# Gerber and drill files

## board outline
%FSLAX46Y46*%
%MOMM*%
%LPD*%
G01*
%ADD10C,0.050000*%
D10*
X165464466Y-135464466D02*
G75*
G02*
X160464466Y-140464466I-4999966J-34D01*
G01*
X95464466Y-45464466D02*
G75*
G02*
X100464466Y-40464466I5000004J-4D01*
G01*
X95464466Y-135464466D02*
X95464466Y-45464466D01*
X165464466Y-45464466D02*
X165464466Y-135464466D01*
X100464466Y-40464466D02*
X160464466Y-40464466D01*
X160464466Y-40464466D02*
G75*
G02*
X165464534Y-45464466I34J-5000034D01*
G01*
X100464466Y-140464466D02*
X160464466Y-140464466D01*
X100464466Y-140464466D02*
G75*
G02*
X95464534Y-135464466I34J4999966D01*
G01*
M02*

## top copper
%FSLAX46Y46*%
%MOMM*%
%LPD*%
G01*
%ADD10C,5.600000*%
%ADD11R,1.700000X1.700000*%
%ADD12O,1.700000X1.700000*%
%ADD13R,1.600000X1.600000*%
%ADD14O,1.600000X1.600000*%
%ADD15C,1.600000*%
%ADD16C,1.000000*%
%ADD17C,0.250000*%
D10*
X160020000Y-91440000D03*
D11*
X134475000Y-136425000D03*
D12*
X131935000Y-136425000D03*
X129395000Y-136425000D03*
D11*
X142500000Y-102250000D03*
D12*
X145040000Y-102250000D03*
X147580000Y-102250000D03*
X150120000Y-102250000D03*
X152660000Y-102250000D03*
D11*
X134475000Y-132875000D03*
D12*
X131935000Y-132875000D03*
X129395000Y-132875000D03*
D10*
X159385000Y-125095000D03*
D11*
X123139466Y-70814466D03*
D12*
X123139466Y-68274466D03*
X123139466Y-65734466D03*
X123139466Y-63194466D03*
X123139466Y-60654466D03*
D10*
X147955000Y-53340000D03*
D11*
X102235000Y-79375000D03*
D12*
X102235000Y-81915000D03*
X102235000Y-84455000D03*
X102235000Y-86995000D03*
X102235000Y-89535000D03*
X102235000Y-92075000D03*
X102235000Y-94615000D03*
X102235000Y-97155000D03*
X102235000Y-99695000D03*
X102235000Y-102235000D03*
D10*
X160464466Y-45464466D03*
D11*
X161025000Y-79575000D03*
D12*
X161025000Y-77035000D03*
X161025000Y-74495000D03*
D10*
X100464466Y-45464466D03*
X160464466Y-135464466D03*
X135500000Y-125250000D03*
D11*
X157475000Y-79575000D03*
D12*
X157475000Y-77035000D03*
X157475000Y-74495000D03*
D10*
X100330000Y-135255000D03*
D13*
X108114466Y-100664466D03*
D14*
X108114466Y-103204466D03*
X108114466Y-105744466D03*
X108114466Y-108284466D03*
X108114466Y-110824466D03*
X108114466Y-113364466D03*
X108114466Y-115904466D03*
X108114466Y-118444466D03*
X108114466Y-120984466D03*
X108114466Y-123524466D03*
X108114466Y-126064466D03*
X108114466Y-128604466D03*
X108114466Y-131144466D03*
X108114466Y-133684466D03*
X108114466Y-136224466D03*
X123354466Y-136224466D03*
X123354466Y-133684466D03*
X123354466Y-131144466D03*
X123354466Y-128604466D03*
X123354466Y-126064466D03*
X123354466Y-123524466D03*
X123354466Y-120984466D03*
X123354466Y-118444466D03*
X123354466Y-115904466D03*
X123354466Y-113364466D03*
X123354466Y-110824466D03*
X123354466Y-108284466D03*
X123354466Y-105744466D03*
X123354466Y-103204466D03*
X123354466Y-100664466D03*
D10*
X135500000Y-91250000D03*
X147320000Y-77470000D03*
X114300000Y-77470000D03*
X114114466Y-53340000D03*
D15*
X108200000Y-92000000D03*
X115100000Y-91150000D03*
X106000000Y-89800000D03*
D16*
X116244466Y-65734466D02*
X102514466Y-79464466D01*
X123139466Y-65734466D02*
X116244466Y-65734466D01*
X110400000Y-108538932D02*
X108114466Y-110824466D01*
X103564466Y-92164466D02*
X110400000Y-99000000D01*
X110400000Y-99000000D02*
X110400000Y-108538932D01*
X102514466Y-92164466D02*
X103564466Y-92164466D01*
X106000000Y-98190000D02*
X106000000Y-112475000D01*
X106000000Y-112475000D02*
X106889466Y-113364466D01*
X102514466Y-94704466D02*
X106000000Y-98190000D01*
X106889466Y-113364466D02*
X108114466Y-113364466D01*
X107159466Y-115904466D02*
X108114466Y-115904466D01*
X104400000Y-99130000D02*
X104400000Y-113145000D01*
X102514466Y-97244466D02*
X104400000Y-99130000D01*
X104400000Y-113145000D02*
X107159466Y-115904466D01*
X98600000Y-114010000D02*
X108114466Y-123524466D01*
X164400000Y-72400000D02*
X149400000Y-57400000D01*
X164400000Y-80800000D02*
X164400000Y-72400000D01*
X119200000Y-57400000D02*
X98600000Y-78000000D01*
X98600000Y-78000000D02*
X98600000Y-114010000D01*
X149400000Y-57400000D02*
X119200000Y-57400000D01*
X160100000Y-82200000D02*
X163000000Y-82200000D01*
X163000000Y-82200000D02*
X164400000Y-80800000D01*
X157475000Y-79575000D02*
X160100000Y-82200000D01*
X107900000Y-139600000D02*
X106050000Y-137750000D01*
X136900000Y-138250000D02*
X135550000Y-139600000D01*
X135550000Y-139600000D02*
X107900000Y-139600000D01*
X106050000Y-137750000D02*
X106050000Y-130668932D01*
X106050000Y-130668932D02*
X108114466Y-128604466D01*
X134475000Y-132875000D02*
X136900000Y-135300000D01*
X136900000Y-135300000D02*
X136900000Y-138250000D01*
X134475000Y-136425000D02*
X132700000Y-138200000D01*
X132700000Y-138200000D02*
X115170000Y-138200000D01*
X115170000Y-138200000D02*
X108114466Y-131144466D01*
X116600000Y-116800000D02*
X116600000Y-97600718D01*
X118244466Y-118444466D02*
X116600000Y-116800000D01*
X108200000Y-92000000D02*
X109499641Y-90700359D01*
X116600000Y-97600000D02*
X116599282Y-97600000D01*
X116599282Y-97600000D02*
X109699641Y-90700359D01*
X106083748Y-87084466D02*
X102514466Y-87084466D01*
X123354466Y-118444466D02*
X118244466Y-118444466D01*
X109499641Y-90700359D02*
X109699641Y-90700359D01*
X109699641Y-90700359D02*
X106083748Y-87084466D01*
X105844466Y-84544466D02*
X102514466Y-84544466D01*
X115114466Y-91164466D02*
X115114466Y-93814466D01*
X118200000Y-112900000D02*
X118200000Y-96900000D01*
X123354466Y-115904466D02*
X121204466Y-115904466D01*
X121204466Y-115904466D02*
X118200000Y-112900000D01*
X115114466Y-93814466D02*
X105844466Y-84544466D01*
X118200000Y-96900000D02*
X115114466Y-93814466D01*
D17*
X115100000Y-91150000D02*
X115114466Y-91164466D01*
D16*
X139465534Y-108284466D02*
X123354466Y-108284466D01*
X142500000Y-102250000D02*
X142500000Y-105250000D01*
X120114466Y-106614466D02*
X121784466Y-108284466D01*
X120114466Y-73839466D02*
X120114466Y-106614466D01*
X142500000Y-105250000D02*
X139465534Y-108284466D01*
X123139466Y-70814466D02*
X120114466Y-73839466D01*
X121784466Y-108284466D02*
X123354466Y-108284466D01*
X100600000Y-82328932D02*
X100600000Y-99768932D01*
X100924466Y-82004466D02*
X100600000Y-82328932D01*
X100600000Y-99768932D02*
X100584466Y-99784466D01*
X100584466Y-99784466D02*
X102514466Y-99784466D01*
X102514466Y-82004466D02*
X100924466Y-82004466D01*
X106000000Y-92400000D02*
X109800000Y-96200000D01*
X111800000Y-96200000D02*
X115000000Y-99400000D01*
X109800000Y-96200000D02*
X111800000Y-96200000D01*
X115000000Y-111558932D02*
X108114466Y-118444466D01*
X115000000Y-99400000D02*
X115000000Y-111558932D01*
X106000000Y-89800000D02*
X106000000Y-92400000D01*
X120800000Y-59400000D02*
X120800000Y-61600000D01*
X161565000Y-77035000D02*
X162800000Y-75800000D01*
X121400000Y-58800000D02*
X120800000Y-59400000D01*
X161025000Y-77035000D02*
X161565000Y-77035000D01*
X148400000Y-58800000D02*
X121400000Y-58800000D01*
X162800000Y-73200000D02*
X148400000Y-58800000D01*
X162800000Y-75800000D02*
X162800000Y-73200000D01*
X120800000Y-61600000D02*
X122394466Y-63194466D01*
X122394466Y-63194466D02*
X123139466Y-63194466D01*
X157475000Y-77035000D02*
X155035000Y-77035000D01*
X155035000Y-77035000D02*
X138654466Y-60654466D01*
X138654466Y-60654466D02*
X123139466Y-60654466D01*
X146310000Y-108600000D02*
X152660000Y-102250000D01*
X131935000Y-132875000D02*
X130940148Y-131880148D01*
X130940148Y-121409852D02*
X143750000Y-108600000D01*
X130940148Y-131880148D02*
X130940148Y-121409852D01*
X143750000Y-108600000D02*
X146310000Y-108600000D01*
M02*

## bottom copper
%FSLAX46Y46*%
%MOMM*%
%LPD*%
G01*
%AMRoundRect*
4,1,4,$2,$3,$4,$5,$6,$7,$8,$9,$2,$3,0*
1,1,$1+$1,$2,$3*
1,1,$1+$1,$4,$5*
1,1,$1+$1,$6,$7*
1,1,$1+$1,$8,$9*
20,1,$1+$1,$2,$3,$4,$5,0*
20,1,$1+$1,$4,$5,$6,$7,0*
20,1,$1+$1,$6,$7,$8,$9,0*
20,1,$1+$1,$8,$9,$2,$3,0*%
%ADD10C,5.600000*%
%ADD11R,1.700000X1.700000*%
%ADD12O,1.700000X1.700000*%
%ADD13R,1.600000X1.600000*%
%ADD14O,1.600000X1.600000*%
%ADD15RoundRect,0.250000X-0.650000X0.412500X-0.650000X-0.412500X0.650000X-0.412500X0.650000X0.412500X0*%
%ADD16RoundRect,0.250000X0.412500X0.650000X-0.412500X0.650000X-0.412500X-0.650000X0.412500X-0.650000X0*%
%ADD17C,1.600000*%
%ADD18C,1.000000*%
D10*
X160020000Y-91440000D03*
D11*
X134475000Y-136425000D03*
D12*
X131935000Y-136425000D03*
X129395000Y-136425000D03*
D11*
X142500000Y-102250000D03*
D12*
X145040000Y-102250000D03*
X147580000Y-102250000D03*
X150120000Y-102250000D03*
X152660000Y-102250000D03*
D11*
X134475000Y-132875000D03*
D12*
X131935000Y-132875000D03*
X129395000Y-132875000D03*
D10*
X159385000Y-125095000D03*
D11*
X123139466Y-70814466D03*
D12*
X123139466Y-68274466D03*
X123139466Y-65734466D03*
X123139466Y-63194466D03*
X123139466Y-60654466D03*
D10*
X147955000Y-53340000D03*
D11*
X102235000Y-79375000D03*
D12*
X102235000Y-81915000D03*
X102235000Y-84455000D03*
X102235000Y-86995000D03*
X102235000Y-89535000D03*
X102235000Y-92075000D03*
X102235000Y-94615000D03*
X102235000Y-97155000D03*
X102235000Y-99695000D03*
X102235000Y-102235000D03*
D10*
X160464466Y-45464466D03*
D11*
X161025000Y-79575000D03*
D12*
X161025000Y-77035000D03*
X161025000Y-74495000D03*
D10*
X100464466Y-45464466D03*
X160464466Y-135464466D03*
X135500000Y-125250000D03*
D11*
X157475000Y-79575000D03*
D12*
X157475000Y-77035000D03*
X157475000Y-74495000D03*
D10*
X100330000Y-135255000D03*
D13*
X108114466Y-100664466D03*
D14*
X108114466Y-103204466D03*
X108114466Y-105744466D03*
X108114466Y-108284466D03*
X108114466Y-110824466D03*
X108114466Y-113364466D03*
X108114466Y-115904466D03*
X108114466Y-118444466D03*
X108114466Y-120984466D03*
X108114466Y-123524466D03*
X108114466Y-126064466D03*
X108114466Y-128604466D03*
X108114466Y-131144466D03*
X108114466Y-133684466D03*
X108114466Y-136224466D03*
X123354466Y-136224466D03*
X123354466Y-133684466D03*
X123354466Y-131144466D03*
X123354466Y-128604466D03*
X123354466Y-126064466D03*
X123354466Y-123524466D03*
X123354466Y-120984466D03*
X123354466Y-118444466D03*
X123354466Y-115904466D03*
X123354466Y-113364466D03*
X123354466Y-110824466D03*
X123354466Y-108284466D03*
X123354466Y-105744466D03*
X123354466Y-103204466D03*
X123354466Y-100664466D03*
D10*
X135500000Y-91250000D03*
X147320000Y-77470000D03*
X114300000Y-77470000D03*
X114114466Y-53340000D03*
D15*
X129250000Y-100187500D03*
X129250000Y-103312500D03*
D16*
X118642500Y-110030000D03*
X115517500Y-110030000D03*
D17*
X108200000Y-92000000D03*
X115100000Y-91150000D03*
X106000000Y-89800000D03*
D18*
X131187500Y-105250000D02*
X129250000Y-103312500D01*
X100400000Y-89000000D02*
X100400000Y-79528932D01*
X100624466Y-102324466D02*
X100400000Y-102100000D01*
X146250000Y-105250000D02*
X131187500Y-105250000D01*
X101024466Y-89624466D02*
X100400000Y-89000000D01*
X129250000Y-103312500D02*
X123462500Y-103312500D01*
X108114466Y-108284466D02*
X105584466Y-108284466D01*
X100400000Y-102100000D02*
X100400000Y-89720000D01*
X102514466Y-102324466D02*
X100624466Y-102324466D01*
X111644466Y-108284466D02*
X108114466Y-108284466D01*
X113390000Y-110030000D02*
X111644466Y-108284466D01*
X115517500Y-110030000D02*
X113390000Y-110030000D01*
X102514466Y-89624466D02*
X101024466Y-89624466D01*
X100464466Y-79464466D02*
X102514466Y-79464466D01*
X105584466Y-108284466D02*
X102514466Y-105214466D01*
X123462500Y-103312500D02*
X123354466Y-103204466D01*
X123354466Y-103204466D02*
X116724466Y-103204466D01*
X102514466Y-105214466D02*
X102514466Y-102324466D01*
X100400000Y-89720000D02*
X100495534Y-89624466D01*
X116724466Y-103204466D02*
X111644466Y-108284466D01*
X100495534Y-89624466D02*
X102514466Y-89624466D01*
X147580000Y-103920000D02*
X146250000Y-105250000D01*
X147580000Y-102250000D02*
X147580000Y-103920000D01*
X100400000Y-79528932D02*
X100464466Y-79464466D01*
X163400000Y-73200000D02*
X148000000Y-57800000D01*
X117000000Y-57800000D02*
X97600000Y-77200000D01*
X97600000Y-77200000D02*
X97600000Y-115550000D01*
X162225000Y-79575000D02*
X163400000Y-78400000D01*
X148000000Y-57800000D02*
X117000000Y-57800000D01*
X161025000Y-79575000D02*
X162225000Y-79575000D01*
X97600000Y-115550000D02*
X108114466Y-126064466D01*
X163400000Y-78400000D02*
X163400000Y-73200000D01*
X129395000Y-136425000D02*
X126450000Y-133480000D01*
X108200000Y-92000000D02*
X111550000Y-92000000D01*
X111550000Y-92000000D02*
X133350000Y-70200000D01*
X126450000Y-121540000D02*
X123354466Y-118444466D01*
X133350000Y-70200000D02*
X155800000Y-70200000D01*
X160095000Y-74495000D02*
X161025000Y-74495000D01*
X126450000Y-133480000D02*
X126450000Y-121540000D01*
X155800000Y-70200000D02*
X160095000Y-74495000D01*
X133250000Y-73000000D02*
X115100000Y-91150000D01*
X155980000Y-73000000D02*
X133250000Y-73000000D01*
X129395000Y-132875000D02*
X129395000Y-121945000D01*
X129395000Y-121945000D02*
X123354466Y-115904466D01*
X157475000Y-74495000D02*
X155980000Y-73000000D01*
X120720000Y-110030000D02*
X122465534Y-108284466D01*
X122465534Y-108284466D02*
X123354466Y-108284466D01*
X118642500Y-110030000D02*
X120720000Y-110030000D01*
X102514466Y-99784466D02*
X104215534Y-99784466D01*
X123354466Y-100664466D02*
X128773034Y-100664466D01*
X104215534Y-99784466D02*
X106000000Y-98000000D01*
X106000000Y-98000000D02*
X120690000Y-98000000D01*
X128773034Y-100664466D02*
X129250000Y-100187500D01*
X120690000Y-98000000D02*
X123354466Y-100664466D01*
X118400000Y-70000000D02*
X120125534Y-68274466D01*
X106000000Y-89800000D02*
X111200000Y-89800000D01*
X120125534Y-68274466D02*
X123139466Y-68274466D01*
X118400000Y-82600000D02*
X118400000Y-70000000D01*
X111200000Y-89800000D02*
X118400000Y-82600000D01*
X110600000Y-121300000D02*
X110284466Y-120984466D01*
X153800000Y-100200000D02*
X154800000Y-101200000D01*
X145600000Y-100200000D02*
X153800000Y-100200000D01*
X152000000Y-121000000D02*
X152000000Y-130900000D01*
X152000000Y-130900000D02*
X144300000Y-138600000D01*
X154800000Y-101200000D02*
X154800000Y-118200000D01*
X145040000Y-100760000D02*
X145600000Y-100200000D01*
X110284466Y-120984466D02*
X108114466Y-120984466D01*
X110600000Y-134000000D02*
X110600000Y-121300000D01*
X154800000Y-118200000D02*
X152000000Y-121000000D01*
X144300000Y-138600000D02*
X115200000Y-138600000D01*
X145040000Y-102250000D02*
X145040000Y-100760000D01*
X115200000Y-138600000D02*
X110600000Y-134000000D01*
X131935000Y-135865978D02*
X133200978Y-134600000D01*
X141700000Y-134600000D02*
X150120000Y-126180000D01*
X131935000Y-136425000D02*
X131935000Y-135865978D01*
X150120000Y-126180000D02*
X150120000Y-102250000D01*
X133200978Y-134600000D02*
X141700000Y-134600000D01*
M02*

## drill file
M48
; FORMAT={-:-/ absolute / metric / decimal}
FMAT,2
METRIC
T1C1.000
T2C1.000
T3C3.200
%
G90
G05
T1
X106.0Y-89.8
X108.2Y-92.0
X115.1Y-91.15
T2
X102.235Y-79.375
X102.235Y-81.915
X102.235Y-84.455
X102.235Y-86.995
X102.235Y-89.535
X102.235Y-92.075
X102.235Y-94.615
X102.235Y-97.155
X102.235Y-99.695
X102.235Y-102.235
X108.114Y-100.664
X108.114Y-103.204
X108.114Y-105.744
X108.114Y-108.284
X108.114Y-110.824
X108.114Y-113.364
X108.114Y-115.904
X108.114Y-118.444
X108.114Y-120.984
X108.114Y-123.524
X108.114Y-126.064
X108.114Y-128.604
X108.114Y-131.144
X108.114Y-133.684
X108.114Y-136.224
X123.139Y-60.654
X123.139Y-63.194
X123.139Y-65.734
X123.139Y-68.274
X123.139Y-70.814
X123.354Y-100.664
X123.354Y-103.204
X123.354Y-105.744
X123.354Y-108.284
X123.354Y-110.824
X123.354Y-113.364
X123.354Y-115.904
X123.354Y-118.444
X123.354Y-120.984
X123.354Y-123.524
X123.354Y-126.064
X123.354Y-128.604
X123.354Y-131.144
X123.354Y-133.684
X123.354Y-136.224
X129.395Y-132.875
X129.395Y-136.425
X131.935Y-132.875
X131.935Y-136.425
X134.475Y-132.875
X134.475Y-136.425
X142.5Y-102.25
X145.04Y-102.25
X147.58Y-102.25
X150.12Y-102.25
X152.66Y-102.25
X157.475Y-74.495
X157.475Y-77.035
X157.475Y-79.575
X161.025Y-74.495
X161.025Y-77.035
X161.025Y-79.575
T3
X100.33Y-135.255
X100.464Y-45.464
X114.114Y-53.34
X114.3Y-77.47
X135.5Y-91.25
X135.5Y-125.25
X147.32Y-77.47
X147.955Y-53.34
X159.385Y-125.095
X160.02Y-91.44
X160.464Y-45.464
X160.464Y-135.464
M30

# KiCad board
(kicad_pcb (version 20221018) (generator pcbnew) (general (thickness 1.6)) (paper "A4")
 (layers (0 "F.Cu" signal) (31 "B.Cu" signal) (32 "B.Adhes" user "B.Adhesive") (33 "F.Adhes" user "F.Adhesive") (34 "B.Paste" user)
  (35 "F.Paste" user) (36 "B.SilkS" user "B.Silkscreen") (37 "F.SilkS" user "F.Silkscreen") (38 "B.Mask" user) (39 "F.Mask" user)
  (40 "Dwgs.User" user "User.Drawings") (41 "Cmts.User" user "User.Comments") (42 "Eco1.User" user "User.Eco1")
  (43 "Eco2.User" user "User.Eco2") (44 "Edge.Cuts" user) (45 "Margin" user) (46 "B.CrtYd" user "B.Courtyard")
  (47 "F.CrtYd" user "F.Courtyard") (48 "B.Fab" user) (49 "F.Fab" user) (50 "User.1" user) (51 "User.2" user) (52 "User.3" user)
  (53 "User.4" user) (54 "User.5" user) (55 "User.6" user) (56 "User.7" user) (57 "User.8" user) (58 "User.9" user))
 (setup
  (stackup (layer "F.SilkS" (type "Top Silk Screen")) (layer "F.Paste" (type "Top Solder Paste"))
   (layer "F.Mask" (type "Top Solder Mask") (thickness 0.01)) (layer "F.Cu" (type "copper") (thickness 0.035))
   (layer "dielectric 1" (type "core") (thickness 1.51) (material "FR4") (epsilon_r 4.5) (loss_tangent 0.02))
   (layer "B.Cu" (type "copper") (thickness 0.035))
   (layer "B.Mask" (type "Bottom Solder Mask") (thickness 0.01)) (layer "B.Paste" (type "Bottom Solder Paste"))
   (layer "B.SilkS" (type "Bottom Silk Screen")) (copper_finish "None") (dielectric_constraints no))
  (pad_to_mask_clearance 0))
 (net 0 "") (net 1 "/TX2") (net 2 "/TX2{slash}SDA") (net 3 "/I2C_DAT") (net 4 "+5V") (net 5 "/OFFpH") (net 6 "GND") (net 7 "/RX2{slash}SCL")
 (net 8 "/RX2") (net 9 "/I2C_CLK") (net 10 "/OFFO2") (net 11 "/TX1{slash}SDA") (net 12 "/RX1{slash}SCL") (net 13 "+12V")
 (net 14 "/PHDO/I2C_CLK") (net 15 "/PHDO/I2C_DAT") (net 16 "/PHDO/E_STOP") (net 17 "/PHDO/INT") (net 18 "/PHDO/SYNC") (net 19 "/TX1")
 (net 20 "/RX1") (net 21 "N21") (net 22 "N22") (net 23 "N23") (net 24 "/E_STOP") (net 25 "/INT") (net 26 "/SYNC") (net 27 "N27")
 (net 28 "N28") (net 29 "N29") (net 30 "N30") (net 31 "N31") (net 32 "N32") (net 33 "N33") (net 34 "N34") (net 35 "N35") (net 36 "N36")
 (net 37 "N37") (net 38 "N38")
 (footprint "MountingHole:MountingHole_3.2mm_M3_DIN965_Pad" (layer "F.Cu") (at 160.02 91.44)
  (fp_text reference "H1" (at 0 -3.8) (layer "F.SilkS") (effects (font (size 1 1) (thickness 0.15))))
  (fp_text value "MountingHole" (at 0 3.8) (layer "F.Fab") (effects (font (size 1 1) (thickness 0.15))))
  (pad "1" thru_hole circle (at 0 0) (size 5.6 5.6) (drill 3.2) (layers "*.Cu" "*.Mask")))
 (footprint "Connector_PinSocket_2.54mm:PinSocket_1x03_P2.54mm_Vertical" (layer "F.Cu") (at 134.475 136.425 -90)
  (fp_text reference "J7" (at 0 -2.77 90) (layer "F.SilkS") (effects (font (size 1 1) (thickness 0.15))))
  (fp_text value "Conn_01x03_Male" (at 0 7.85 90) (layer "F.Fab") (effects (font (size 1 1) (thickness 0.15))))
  (pad "1" thru_hole rect (at 0 0 270) (size 1.7 1.7) (drill 1) (layers "*.Cu" "*.Mask") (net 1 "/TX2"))
  (pad "2" thru_hole oval (at 0 2.54 270) (size 1.7 1.7) (drill 1) (layers "*.Cu" "*.Mask") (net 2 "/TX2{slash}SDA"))
  (pad "3" thru_hole oval (at 0 5.08 270) (size 1.7 1.7) (drill 1) (layers "*.Cu" "*.Mask") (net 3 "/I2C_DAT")))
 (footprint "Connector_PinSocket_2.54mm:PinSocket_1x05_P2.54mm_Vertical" (layer "F.Cu") (at 142.5 102.25 90)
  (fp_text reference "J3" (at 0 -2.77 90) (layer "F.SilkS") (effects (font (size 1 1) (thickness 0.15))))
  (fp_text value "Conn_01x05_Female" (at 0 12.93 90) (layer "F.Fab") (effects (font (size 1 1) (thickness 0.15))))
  (pad "1" thru_hole rect (at 0 0 90) (size 1.7 1.7) (drill 1) (layers "*.Cu" "*.Mask") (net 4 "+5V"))
  (pad "2" thru_hole oval (at 0 2.54 90) (size 1.7 1.7) (drill 1) (layers "*.Cu" "*.Mask") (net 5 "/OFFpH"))
  (pad "3" thru_hole oval (at 0 5.08 90) (size 1.7 1.7) (drill 1) (layers "*.Cu" "*.Mask") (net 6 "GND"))
  (pad "4" thru_hole oval (at 0 7.62 90) (size 1.7 1.7) (drill 1) (layers "*.Cu" "*.Mask") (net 2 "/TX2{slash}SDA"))
  (pad "5" thru_hole oval (at 0 10.16 90) (size 1.7 1.7) (drill 1) (layers "*.Cu" "*.Mask") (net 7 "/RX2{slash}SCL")))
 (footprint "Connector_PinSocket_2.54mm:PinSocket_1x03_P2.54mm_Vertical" (layer "F.Cu") (at 134.475 132.875 -90)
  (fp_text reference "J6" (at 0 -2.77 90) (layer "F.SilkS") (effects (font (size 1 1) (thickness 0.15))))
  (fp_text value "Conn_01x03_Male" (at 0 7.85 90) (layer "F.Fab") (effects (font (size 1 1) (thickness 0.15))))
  (pad "1" thru_hole rect (at 0 0 270) (size 1.7 1.7) (drill 1) (layers "*.Cu" "*.Mask") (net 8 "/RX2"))
  (pad "2" thru_hole oval (at 0 2.54 270) (size 1.7 1.7) (drill 1) (layers "*.Cu" "*.Mask") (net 7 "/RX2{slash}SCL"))
  (pad "3" thru_hole oval (at 0 5.08 270) (size 1.7 1.7) (drill 1) (layers "*.Cu" "*.Mask") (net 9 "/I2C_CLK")))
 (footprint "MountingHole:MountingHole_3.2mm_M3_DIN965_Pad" (layer "F.Cu") (at 159.385 125.095)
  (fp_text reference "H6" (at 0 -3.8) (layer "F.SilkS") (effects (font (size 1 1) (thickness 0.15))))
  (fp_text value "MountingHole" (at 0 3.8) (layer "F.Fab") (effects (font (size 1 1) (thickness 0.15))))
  (pad "1" thru_hole circle (at 0 0) (size 5.6 5.6) (drill 3.2) (layers "*.Cu" "*.Mask")))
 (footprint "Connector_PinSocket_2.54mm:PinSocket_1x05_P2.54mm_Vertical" (layer "F.Cu") (at 123.139466 70.814466 180)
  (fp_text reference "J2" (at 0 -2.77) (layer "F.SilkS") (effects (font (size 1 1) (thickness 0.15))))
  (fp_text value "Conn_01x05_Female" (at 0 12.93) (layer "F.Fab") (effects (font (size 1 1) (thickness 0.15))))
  (pad "1" thru_hole rect (at 0 0 180) (size 1.7 1.7) (drill 1) (layers "*.Cu" "*.Mask") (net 4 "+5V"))
  (pad "2" thru_hole oval (at 0 2.54 180) (size 1.7 1.7) (drill 1) (layers "*.Cu" "*.Mask") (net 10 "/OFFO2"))
  (pad "3" thru_hole oval (at 0 5.08 180) (size 1.7 1.7) (drill 1) (layers "*.Cu" "*.Mask") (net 6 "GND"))
  (pad "4" thru_hole oval (at 0 7.62 180) (size 1.7 1.7) (drill 1) (layers "*.Cu" "*.Mask") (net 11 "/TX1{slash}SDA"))
  (pad "5" thru_hole oval (at 0 10.16 180) (size 1.7 1.7) (drill 1) (layers "*.Cu" "*.Mask") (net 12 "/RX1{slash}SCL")))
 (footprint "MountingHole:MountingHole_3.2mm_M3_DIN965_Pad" (layer "F.Cu") (at 147.955 53.34)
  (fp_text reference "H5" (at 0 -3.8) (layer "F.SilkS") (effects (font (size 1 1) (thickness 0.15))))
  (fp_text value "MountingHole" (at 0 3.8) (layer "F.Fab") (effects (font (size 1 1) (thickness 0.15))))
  (pad "1" thru_hole circle (at 0 0) (size 5.6 5.6) (drill 3.2) (layers "*.Cu" "*.Mask")))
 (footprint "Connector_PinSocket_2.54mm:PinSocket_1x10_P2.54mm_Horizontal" (layer "F.Cu") (at 102.235 79.375)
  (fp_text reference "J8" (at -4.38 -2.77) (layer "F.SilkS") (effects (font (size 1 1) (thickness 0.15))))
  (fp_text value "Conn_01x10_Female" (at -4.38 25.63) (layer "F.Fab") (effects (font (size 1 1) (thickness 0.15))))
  (pad "1" thru_hole rect (at 0 0) (size 1.7 1.7) (drill 1) (layers "*.Cu" "*.Mask") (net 6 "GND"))
  (pad "2" thru_hole oval (at 0 2.54) (size 1.7 1.7) (drill 1) (layers "*.Cu" "*.Mask") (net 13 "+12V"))
  (pad "3" thru_hole oval (at 0 5.08) (size 1.7 1.7) (drill 1) (layers "*.Cu" "*.Mask") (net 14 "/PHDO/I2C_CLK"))
  (pad "4" thru_hole oval (at 0 7.62) (size 1.7 1.7) (drill 1) (layers "*.Cu" "*.Mask") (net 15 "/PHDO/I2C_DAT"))
  (pad "5" thru_hole oval (at 0 10.16) (size 1.7 1.7) (drill 1) (layers "*.Cu" "*.Mask") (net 6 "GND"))
  (pad "6" thru_hole oval (at 0 12.7) (size 1.7 1.7) (drill 1) (layers "*.Cu" "*.Mask") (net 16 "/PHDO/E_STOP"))
  (pad "7" thru_hole oval (at 0 15.24) (size 1.7 1.7) (drill 1) (layers "*.Cu" "*.Mask") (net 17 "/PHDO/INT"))
  (pad "8" thru_hole oval (at 0 17.78) (size 1.7 1.7) (drill 1) (layers "*.Cu" "*.Mask") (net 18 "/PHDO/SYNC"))
  (pad "9" thru_hole oval (at 0 20.32) (size 1.7 1.7) (drill 1) (layers "*.Cu" "*.Mask") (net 13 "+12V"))
  (pad "10" thru_hole oval (at 0 22.86) (size 1.7 1.7) (drill 1) (layers "*.Cu" "*.Mask") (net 6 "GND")))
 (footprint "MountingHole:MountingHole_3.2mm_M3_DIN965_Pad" (layer "F.Cu") (at 160.464466 45.464466)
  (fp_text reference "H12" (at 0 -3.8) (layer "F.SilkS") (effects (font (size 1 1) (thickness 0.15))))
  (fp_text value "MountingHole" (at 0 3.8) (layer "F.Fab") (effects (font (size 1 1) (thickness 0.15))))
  (pad "1" thru_hole circle (at 0 0) (size 5.6 5.6) (drill 3.2) (layers "*.Cu" "*.Mask")))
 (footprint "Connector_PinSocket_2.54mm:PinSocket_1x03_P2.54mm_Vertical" (layer "F.Cu") (at 161.025 79.575 180)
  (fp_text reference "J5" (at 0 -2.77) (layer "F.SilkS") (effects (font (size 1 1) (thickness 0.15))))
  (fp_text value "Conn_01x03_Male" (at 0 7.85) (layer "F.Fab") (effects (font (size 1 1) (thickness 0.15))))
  (pad "1" thru_hole rect (at 0 0 180) (size 1.7 1.7) (drill 1) (layers "*.Cu" "*.Mask") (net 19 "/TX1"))
  (pad "2" thru_hole oval (at 0 2.54 180) (size 1.7 1.7) (drill 1) (layers "*.Cu" "*.Mask") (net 11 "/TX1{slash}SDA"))
  (pad "3" thru_hole oval (at 0 5.08 180) (size 1.7 1.7) (drill 1) (layers "*.Cu" "*.Mask") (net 3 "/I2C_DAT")))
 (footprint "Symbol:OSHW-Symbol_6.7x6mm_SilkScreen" (layer "F.Cu") (at 109.515 44.979 180)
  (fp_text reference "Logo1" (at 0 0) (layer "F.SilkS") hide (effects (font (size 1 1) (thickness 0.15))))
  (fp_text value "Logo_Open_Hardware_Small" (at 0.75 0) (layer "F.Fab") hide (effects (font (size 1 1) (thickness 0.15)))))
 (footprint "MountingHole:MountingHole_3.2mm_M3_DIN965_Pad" (layer "F.Cu") (at 100.464466 45.464466)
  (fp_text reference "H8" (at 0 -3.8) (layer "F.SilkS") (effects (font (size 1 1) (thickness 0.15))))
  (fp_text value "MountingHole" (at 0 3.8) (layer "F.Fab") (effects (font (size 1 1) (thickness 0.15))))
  (pad "1" thru_hole circle (at 0 0) (size 5.6 5.6) (drill 3.2) (layers "*.Cu" "*.Mask")))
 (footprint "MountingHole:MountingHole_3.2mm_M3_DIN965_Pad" (layer "F.Cu") (at 160.464466 135.464466)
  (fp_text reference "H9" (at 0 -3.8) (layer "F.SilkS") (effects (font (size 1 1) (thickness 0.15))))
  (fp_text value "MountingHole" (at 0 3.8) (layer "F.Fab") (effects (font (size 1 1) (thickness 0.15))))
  (pad "1" thru_hole circle (at 0 0) (size 5.6 5.6) (drill 3.2) (layers "*.Cu" "*.Mask")))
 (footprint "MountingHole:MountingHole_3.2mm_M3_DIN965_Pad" (layer "F.Cu") (at 135.5 125.25 90)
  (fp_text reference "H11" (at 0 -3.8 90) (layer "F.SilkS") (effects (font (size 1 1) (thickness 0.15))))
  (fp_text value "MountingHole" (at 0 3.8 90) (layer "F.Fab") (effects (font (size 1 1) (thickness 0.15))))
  (pad "1" thru_hole circle (at 0 0 90) (size 5.6 5.6) (drill 3.2) (layers "*.Cu" "*.Mask")))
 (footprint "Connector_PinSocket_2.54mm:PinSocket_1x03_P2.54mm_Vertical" (layer "F.Cu") (at 157.475 79.575 180)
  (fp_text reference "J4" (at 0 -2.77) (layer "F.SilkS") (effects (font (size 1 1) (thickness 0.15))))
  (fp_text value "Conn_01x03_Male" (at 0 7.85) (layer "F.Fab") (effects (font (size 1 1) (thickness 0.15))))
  (pad "1" thru_hole rect (at 0 0 180) (size 1.7 1.7) (drill 1) (layers "*.Cu" "*.Mask") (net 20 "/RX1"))
  (pad "2" thru_hole oval (at 0 2.54 180) (size 1.7 1.7) (drill 1) (layers "*.Cu" "*.Mask") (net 12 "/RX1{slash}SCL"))
  (pad "3" thru_hole oval (at 0 5.08 180) (size 1.7 1.7) (drill 1) (layers "*.Cu" "*.Mask") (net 9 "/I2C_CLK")))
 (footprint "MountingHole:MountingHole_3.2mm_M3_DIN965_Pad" (layer "F.Cu") (at 100.33 135.255)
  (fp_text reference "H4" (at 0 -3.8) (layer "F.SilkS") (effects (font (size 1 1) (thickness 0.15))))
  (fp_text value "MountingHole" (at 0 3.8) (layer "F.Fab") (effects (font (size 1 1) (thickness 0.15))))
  (pad "1" thru_hole circle (at 0 0) (size 5.6 5.6) (drill 3.2) (layers "*.Cu" "*.Mask")))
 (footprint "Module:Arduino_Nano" (layer "F.Cu") (at 108.114466 100.664466)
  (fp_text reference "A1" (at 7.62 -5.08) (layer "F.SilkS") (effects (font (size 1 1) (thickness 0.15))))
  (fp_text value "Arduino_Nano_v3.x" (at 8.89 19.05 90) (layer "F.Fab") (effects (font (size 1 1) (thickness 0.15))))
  (pad "1" thru_hole rect (at 0 0) (size 1.6 1.6) (drill 1) (layers "*.Cu" "*.Mask") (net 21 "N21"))
  (pad "2" thru_hole oval (at 0 2.54) (size 1.6 1.6) (drill 1) (layers "*.Cu" "*.Mask") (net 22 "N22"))
  (pad "3" thru_hole oval (at 0 5.08) (size 1.6 1.6) (drill 1) (layers "*.Cu" "*.Mask") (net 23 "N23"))
  (pad "4" thru_hole oval (at 0 7.62) (size 1.6 1.6) (drill 1) (layers "*.Cu" "*.Mask") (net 6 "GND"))
  (pad "5" thru_hole oval (at 0 10.16) (size 1.6 1.6) (drill 1) (layers "*.Cu" "*.Mask") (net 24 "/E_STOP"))
  (pad "6" thru_hole oval (at 0 12.7) (size 1.6 1.6) (drill 1) (layers "*.Cu" "*.Mask") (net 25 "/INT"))
  (pad "7" thru_hole oval (at 0 15.24) (size 1.6 1.6) (drill 1) (layers "*.Cu" "*.Mask") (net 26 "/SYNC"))
  (pad "8" thru_hole oval (at 0 17.78) (size 1.6 1.6) (drill 1) (layers "*.Cu" "*.Mask") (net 10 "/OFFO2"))
  (pad "9" thru_hole oval (at 0 20.32) (size 1.6 1.6) (drill 1) (layers "*.Cu" "*.Mask") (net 5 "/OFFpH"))
  (pad "10" thru_hole oval (at 0 22.86) (size 1.6 1.6) (drill 1) (layers "*.Cu" "*.Mask") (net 20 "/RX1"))
  (pad "11" thru_hole oval (at 0 25.4) (size 1.6 1.6) (drill 1) (layers "*.Cu" "*.Mask") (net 19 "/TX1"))
  (pad "12" thru_hole oval (at 0 27.94) (size 1.6 1.6) (drill 1) (layers "*.Cu" "*.Mask") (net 8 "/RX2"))
  (pad "13" thru_hole oval (at 0 30.48) (size 1.6 1.6) (drill 1) (layers "*.Cu" "*.Mask") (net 1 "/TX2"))
  (pad "14" thru_hole oval (at 0 33.02) (size 1.6 1.6) (drill 1) (layers "*.Cu" "*.Mask") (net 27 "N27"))
  (pad "15" thru_hole oval (at 0 35.56) (size 1.6 1.6) (drill 1) (layers "*.Cu" "*.Mask") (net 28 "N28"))
  (pad "16" thru_hole oval (at 15.24 35.56) (size 1.6 1.6) (drill 1) (layers "*.Cu" "*.Mask") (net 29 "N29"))
  (pad "17" thru_hole oval (at 15.24 33.02) (size 1.6 1.6) (drill 1) (layers "*.Cu" "*.Mask") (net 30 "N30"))
  (pad "18" thru_hole oval (at 15.24 30.48) (size 1.6 1.6) (drill 1) (layers "*.Cu" "*.Mask") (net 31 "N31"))
  (pad "19" thru_hole oval (at 15.24 27.94) (size 1.6 1.6) (drill 1) (layers "*.Cu" "*.Mask") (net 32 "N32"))
  (pad "20" thru_hole oval (at 15.24 25.4) (size 1.6 1.6) (drill 1) (layers "*.Cu" "*.Mask") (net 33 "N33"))
  (pad "21" thru_hole oval (at 15.24 22.86) (size 1.6 1.6) (drill 1) (layers "*.Cu" "*.Mask") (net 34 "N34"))
  (pad "22" thru_hole oval (at 15.24 20.32) (size 1.6 1.6) (drill 1) (layers "*.Cu" "*.Mask") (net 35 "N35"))
  (pad "23" thru_hole oval (at 15.24 17.78) (size 1.6 1.6) (drill 1) (layers "*.Cu" "*.Mask") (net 3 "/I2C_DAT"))
  (pad "24" thru_hole oval (at 15.24 15.24) (size 1.6 1.6) (drill 1) (layers "*.Cu" "*.Mask") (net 9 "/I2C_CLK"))
  (pad "25" thru_hole oval (at 15.24 12.7) (size 1.6 1.6) (drill 1) (layers "*.Cu" "*.Mask") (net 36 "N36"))
  (pad "26" thru_hole oval (at 15.24 10.16) (size 1.6 1.6) (drill 1) (layers "*.Cu" "*.Mask") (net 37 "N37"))
  (pad "27" thru_hole oval (at 15.24 7.62) (size 1.6 1.6) (drill 1) (layers "*.Cu" "*.Mask") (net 4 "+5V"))
  (pad "28" thru_hole oval (at 15.24 5.08) (size 1.6 1.6) (drill 1) (layers "*.Cu" "*.Mask") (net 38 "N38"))
  (pad "29" thru_hole oval (at 15.24 2.54) (size 1.6 1.6) (drill 1) (layers "*.Cu" "*.Mask") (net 6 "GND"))
  (pad "30" thru_hole oval (at 15.24 0) (size 1.6 1.6) (drill 1) (layers "*.Cu" "*.Mask") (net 13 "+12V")))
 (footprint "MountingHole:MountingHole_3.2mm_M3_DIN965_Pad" (layer "F.Cu") (at 135.5 91.25 90)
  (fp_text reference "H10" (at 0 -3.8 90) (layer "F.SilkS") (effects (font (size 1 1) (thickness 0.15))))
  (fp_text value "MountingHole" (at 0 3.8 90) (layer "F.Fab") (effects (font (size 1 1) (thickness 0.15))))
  (pad "1" thru_hole circle (at 0 0 90) (size 5.6 5.6) (drill 3.2) (layers "*.Cu" "*.Mask")))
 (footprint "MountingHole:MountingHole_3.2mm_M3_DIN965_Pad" (layer "F.Cu") (at 147.32 77.47)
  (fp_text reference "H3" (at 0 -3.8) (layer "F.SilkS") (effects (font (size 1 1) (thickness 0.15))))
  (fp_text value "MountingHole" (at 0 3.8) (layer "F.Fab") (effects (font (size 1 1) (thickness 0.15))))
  (pad "1" thru_hole circle (at 0 0) (size 5.6 5.6) (drill 3.2) (layers "*.Cu" "*.Mask")))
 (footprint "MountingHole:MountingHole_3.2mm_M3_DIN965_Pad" (layer "F.Cu") (at 114.3 77.47)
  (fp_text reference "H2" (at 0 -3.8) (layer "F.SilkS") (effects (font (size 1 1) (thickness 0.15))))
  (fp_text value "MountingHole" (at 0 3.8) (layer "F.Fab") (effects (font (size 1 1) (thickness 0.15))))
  (pad "1" thru_hole circle (at 0 0) (size 5.6 5.6) (drill 3.2) (layers "*.Cu" "*.Mask")))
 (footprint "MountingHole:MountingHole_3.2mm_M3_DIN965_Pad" (layer "F.Cu") (at 114.114466 53.34)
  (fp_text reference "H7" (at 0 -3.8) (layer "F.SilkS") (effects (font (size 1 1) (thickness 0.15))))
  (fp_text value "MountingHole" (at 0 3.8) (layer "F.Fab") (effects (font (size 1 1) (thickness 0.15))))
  (pad "1" thru_hole circle (at 0 0) (size 5.6 5.6) (drill 3.2) (layers "*.Cu" "*.Mask")))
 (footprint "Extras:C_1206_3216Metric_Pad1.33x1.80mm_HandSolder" (layer "B.Cu") (at 129.25 101.75 -90)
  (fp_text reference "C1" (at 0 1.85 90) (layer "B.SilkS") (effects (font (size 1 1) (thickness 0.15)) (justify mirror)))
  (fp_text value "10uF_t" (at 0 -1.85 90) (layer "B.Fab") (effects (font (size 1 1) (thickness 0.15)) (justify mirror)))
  (pad "1" smd roundrect (at -1.5625 0 270) (size 1.325 1.8) (layers "B.Cu" "B.Paste" "B.Mask") (roundrect_rratio 0.1886792453)
   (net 13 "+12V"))
  (pad "2" smd roundrect (at 1.5625 0 270) (size 1.325 1.8) (layers "B.Cu" "B.Paste" "B.Mask") (roundrect_rratio 0.1886792453) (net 6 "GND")))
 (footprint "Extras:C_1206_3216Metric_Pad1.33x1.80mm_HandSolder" (layer "B.Cu") (at 117.08 110.03 180)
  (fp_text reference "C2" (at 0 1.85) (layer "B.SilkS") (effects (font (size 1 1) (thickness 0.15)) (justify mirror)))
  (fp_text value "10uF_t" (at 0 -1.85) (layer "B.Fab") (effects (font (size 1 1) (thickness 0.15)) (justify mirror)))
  (pad "1" smd roundrect (at -1.5625 0 180) (size 1.325 1.8) (layers "B.Cu" "B.Paste" "B.Mask") (roundrect_rratio 0.1886792453)
   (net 4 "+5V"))
  (pad "2" smd roundrect (at 1.5625 0 180) (size 1.325 1.8) (layers "B.Cu" "B.Paste" "B.Mask") (roundrect_rratio 0.1886792453) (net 6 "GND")))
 (gr_arc (start 165.464466 135.464466) (mid 164 139) (end 160.464466 140.464466) (stroke (width 0.05) (type solid)) (layer "Edge.Cuts"))
 (gr_arc (start 95.464466 45.464466) (mid 96.928932 41.928932) (end 100.464466 40.464466) (stroke (width 0.05) (type solid))
  (layer "Edge.Cuts"))
 (gr_line (start 95.464466 135.464466) (end 95.464466 45.464466) (stroke (width 0.05) (type solid)) (layer "Edge.Cuts"))
 (gr_line (start 165.464466 45.464466) (end 165.464466 135.464466) (stroke (width 0.05) (type solid)) (layer "Edge.Cuts"))
 (gr_line (start 100.464466 40.464466) (end 160.464466 40.464466) (stroke (width 0.05) (type solid)) (layer "Edge.Cuts"))
 (gr_arc (start 160.464466 40.464466) (mid 164 41.928932) (end 165.464466 45.464466) (stroke (width 0.05) (type solid)) (layer "Edge.Cuts"))
 (gr_line (start 100.464466 140.464466) (end 160.464466 140.464466) (stroke (width 0.05) (type solid)) (layer "Edge.Cuts"))
 (gr_arc (start 100.464466 140.464466) (mid 96.928932 139) (end 95.464466 135.464466) (stroke (width 0.05) (type solid)) (layer "Edge.Cuts"))
 (segment (start 116.244466 65.734466) (end 102.514466 79.464466) (width 1) (layer "F.Cu") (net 6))
 (segment (start 123.139466 65.734466) (end 116.244466 65.734466) (width 1) (layer "F.Cu") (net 6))
 (segment (start 131.1875 105.25) (end 129.25 103.3125) (width 1) (layer "B.Cu") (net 6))
 (segment (start 100.4 89) (end 100.4 79.528932) (width 1) (layer "B.Cu") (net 6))
 (segment (start 100.624466 102.324466) (end 100.4 102.1) (width 1) (layer "B.Cu") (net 6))
 (segment (start 146.25 105.25) (end 131.1875 105.25) (width 1) (layer "B.Cu") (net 6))
 (segment (start 101.024466 89.624466) (end 100.4 89) (width 1) (layer "B.Cu") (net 6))
 (segment (start 129.25 103.3125) (end 123.4625 103.3125) (width 1) (layer "B.Cu") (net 6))
 (segment (start 108.114466 108.284466) (end 105.584466 108.284466) (width 1) (layer "B.Cu") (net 6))
 (segment (start 100.4 102.1) (end 100.4 89.72) (width 1) (layer "B.Cu") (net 6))
 (segment (start 102.514466 102.324466) (end 100.624466 102.324466) (width 1) (layer "B.Cu") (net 6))
 (segment (start 111.644466 108.284466) (end 108.114466 108.284466) (width 1) (layer "B.Cu") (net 6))
 (segment (start 113.39 110.03) (end 111.644466 108.284466) (width 1) (layer "B.Cu") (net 6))
 (segment (start 115.5175 110.03) (end 113.39 110.03) (width 1) (layer "B.Cu") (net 6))
 (segment (start 102.514466 89.624466) (end 101.024466 89.624466) (width 1) (layer "B.Cu") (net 6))
 (segment (start 100.464466 79.464466) (end 102.514466 79.464466) (width 1) (layer "B.Cu") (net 6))
 (segment (start 105.584466 108.284466) (end 102.514466 105.214466) (width 1) (layer "B.Cu") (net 6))
 (segment (start 123.4625 103.3125) (end 123.354466 103.204466) (width 1) (layer "B.Cu") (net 6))
 (segment (start 123.354466 103.204466) (end 116.724466 103.204466) (width 1) (layer "B.Cu") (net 6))
 (segment (start 102.514466 105.214466) (end 102.514466 102.324466) (width 1) (layer "B.Cu") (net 6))
 (segment (start 100.4 89.72) (end 100.495534 89.624466) (width 1) (layer "B.Cu") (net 6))
 (segment (start 116.724466 103.204466) (end 111.644466 108.284466) (width 1) (layer "B.Cu") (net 6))
 (segment (start 100.495534 89.624466) (end 102.514466 89.624466) (width 1) (layer "B.Cu") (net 6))
 (segment (start 147.58 103.92) (end 146.25 105.25) (width 1) (layer "B.Cu") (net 6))
 (segment (start 147.58 102.25) (end 147.58 103.92) (width 1) (layer "B.Cu") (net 6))
 (segment (start 100.4 79.528932) (end 100.464466 79.464466) (width 1) (layer "B.Cu") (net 6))
 (segment (start 110.4 108.538932) (end 108.114466 110.824466) (width 1) (layer "F.Cu") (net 24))
 (segment (start 103.564466 92.164466) (end 110.4 99) (width 1) (layer "F.Cu") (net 24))
 (segment (start 110.4 99) (end 110.4 108.538932) (width 1) (layer "F.Cu") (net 24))
 (segment (start 102.514466 92.164466) (end 103.564466 92.164466) (width 1) (layer "F.Cu") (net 24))
 (segment (start 106 98.19) (end 106 112.475) (width 1) (layer "F.Cu") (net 25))
 (segment (start 106 112.475) (end 106.889466 113.364466) (width 1) (layer "F.Cu") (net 25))
 (segment (start 102.514466 94.704466) (end 106 98.19) (width 1) (layer "F.Cu") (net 25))
 (segment (start 106.889466 113.364466) (end 108.114466 113.364466) (width 1) (layer "F.Cu") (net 25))
 (segment (start 107.159466 115.904466) (end 108.114466 115.904466) (width 1) (layer "F.Cu") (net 26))
 (segment (start 104.4 99.13) (end 104.4 113.145) (width 1) (layer "F.Cu") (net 26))
 (segment (start 102.514466 97.244466) (end 104.4 99.13) (width 1) (layer "F.Cu") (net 26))
 (segment (start 104.4 113.145) (end 107.159466 115.904466) (width 1) (layer "F.Cu") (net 26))
 (segment (start 98.6 114.01) (end 108.114466 123.524466) (width 1) (layer "F.Cu") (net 20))
 (segment (start 164.4 72.4) (end 149.4 57.4) (width 1) (layer "F.Cu") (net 20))
 (segment (start 164.4 80.8) (end 164.4 72.4) (width 1) (layer "F.Cu") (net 20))
 (segment (start 119.2 57.4) (end 98.6 78) (width 1) (layer "F.Cu") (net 20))
 (segment (start 98.6 78) (end 98.6 114.01) (width 1) (layer "F.Cu") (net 20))
 (segment (start 149.4 57.4) (end 119.2 57.4) (width 1) (layer "F.Cu") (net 20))
 (segment (start 160.1 82.2) (end 163 82.2) (width 1) (layer "F.Cu") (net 20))
 (segment (start 163 82.2) (end 164.4 80.8) (width 1) (layer "F.Cu") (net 20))
 (segment (start 157.475 79.575) (end 160.1 82.2) (width 1) (layer "F.Cu") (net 20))
 (segment (start 163.4 73.2) (end 148 57.8) (width 1) (layer "B.Cu") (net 19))
 (segment (start 117 57.8) (end 97.6 77.2) (width 1) (layer "B.Cu") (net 19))
 (segment (start 97.6 77.2) (end 97.6 115.55) (width 1) (layer "B.Cu") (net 19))
 (segment (start 162.225 79.575) (end 163.4 78.4) (width 1) (layer "B.Cu") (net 19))
 (segment (start 148 57.8) (end 117 57.8) (width 1) (layer "B.Cu") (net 19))
 (segment (start 161.025 79.575) (end 162.225 79.575) (width 1) (layer "B.Cu") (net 19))
 (segment (start 97.6 115.55) (end 108.114466 126.064466) (width 1) (layer "B.Cu") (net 19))
 (segment (start 163.4 78.4) (end 163.4 73.2) (width 1) (layer "B.Cu") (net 19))
 (segment (start 107.9 139.6) (end 106.05 137.75) (width 1) (layer "F.Cu") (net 8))
 (segment (start 136.9 138.25) (end 135.55 139.6) (width 1) (layer "F.Cu") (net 8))
 (segment (start 135.55 139.6) (end 107.9 139.6) (width 1) (layer "F.Cu") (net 8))
 (segment (start 106.05 137.75) (end 106.05 130.668932) (width 1) (layer "F.Cu") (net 8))
 (segment (start 106.05 130.668932) (end 108.114466 128.604466) (width 1) (layer "F.Cu") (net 8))
 (segment (start 134.475 132.875) (end 136.9 135.3) (width 1) (layer "F.Cu") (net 8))
 (segment (start 136.9 135.3) (end 136.9 138.25) (width 1) (layer "F.Cu") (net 8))
 (segment (start 134.475 136.425) (end 132.7 138.2) (width 1) (layer "F.Cu") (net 1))
 (segment (start 132.7 138.2) (end 115.17 138.2) (width 1) (layer "F.Cu") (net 1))
 (segment (start 115.17 138.2) (end 108.114466 131.144466) (width 1) (layer "F.Cu") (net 1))
 (segment (start 116.6 116.8) (end 116.6 97.600718) (width 1) (layer "F.Cu") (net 3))
 (segment (start 118.244466 118.444466) (end 116.6 116.8) (width 1) (layer "F.Cu") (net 3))
 (segment (start 108.2 92) (end 109.499641 90.700359) (width 1) (layer "F.Cu") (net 3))
 (segment (start 116.6 97.6) (end 116.599282 97.6) (width 1) (layer "F.Cu") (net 3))
 (segment (start 116.599282 97.6) (end 109.699641 90.700359) (width 1) (layer "F.Cu") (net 3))
 (segment (start 106.083748 87.084466) (end 102.514466 87.084466) (width 1) (layer "F.Cu") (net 3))
 (segment (start 123.354466 118.444466) (end 118.244466 118.444466) (width 1) (layer "F.Cu") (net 3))
 (segment (start 109.499641 90.700359) (end 109.699641 90.700359) (width 1) (layer "F.Cu") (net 3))
 (segment (start 109.699641 90.700359) (end 106.083748 87.084466) (width 1) (layer "F.Cu") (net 3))
 (via (at 108.2 92) (size 1.6) (drill 1) (layers "F.Cu" "B.Cu") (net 3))
 (segment (start 129.395 136.425) (end 126.45 133.48) (width 1) (layer "B.Cu") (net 3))
 (segment (start 108.2 92) (end 111.55 92) (width 1) (layer "B.Cu") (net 3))
 (segment (start 111.55 92) (end 133.35 70.2) (width 1) (layer "B.Cu") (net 3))
 (segment (start 126.45 121.54) (end 123.354466 118.444466) (width 1) (layer "B.Cu") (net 3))
 (segment (start 133.35 70.2) (end 155.8 70.2) (width 1) (layer "B.Cu") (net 3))
 (segment (start 160.095 74.495) (end 161.025 74.495) (width 1) (layer "B.Cu") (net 3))
 (segment (start 126.45 133.48) (end 126.45 121.54) (width 1) (layer "B.Cu") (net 3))
 (segment (start 155.8 70.2) (end 160.095 74.495) (width 1) (layer "B.Cu") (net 3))
 (segment (start 105.844466 84.544466) (end 102.514466 84.544466) (width 1) (layer "F.Cu") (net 9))
 (segment (start 115.114466 91.164466) (end 115.114466 93.814466) (width 1) (layer "F.Cu") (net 9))
 (segment (start 118.2 112.9) (end 118.2 96.9) (width 1) (layer "F.Cu") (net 9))
 (segment (start 123.354466 115.904466) (end 121.204466 115.904466) (width 1) (layer "F.Cu") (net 9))
 (segment (start 121.204466 115.904466) (end 118.2 112.9) (width 1) (layer "F.Cu") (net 9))
 (segment (start 115.114466 93.814466) (end 105.844466 84.544466) (width 1) (layer "F.Cu") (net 9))
 (segment (start 118.2 96.9) (end 115.114466 93.814466) (width 1) (layer "F.Cu") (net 9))
 (segment (start 115.1 91.15) (end 115.114466 91.164466) (width 0.25) (layer "F.Cu") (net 9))
 (via (at 115.1 91.15) (size 1.6) (drill 1) (layers "F.Cu" "B.Cu") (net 9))
 (segment (start 133.25 73) (end 115.1 91.15) (width 1) (layer "B.Cu") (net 9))
 (segment (start 155.98 73) (end 133.25 73) (width 1) (layer "B.Cu") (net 9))
 (segment (start 129.395 132.875) (end 129.395 121.945) (width 1) (layer "B.Cu") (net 9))
 (segment (start 129.395 121.945) (end 123.354466 115.904466) (width 1) (layer "B.Cu") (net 9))
 (segment (start 157.475 74.495) (end 155.98 73) (width 1) (layer "B.Cu") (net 9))
 (segment (start 139.465534 108.284466) (end 123.354466 108.284466) (width 1) (layer "F.Cu") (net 4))
 (segment (start 142.5 102.25) (end 142.5 105.25) (width 1) (layer "F.Cu") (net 4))
 (segment (start 120.114466 106.614466) (end 121.784466 108.284466) (width 1) (layer "F.Cu") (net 4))
 (segment (start 120.114466 73.839466) (end 120.114466 106.614466) (width 1) (layer "F.Cu") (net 4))
 (segment (start 142.5 105.25) (end 139.465534 108.284466) (width 1) (layer "F.Cu") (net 4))
 (segment (start 123.139466 70.814466) (end 120.114466 73.839466) (width 1) (layer "F.Cu") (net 4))
 (segment (start 121.784466 108.284466) (end 123.354466 108.284466) (width 1) (layer "F.Cu") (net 4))
 (segment (start 120.72 110.03) (end 122.465534 108.284466) (width 1) (layer "B.Cu") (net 4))
 (segment (start 122.465534 108.284466) (end 123.354466 108.284466) (width 1) (layer "B.Cu") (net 4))
 (segment (start 118.6425 110.03) (end 120.72 110.03) (width 1) (layer "B.Cu") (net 4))
 (segment (start 100.6 82.328932) (end 100.6 99.768932) (width 1) (layer "F.Cu") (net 13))
 (segment (start 100.924466 82.004466) (end 100.6 82.328932) (width 1) (layer "F.Cu") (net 13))
 (segment (start 100.6 99.768932) (end 100.584466 99.784466) (width 1) (layer "F.Cu") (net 13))
 (segment (start 100.584466 99.784466) (end 102.514466 99.784466) (width 1) (layer "F.Cu") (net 13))
 (segment (start 102.514466 82.004466) (end 100.924466 82.004466) (width 1) (layer "F.Cu") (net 13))
 (segment (start 102.514466 99.784466) (end 104.215534 99.784466) (width 1) (layer "B.Cu") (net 13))
 (segment (start 123.354466 100.664466) (end 128.773034 100.664466) (width 1) (layer "B.Cu") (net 13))
 (segment (start 104.215534 99.784466) (end 106 98) (width 1) (layer "B.Cu") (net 13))
 (segment (start 106 98) (end 120.69 98) (width 1) (layer "B.Cu") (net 13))
 (segment (start 128.773034 100.664466) (end 129.25 100.1875) (width 1) (layer "B.Cu") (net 13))
 (segment (start 120.69 98) (end 123.354466 100.664466) (width 1) (layer "B.Cu") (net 13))
 (segment (start 106 92.4) (end 109.8 96.2) (width 1) (layer "F.Cu") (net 10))
 (segment (start 111.8 96.2) (end 115 99.4) (width 1) (layer "F.Cu") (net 10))
 (segment (start 109.8 96.2) (end 111.8 96.2) (width 1) (layer "F.Cu") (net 10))
 (segment (start 115 111.558932) (end 108.114466 118.444466) (width 1) (layer "F.Cu") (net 10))
 (segment (start 115 99.4) (end 115 111.558932) (width 1) (layer "F.Cu") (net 10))
 (segment (start 106 89.8) (end 106 92.4) (width 1) (layer "F.Cu") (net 10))
 (via (at 106 89.8) (size 1.6) (drill 1) (layers "F.Cu" "B.Cu") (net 10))
 (segment (start 118.4 70) (end 120.125534 68.274466) (width 1) (layer "B.Cu") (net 10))
 (segment (start 106 89.8) (end 111.2 89.8) (width 1) (layer "B.Cu") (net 10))
 (segment (start 120.125534 68.274466) (end 123.139466 68.274466) (width 1) (layer "B.Cu") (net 10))
 (segment (start 118.4 82.6) (end 118.4 70) (width 1) (layer "B.Cu") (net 10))
 (segment (start 111.2 89.8) (end 118.4 82.6) (width 1) (layer "B.Cu") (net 10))
 (segment (start 110.6 121.3) (end 110.284466 120.984466) (width 1) (layer "B.Cu") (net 5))
 (segment (start 153.8 100.2) (end 154.8 101.2) (width 1) (layer "B.Cu") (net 5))
 (segment (start 145.6 100.2) (end 153.8 100.2) (width 1) (layer "B.Cu") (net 5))
 (segment (start 152 121) (end 152 130.9) (width 1) (layer "B.Cu") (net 5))
 (segment (start 152 130.9) (end 144.3 138.6) (width 1) (layer "B.Cu") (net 5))
 (segment (start 154.8 101.2) (end 154.8 118.2) (width 1) (layer "B.Cu") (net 5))
 (segment (start 145.04 100.76) (end 145.6 100.2) (width 1) (layer "B.Cu") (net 5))
 (segment (start 110.284466 120.984466) (end 108.114466 120.984466) (width 1) (layer "B.Cu") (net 5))
 (segment (start 110.6 134) (end 110.6 121.3) (width 1) (layer "B.Cu") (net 5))
 (segment (start 154.8 118.2) (end 152 121) (width 1) (layer "B.Cu") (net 5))
 (segment (start 144.3 138.6) (end 115.2 138.6) (width 1) (layer "B.Cu") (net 5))
 (segment (start 145.04 102.25) (end 145.04 100.76) (width 1) (layer "B.Cu") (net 5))
 (segment (start 115.2 138.6) (end 110.6 134) (width 1) (layer "B.Cu") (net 5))
 (segment (start 120.8 59.4) (end 120.8 61.6) (width 1) (layer "F.Cu") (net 11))
 (segment (start 161.565 77.035) (end 162.8 75.8) (width 1) (layer "F.Cu") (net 11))
 (segment (start 121.4 58.8) (end 120.8 59.4) (width 1) (layer "F.Cu") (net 11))
 (segment (start 161.025 77.035) (end 161.565 77.035) (width 1) (layer "F.Cu") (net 11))
 (segment (start 148.4 58.8) (end 121.4 58.8) (width 1) (layer "F.Cu") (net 11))
 (segment (start 162.8 73.2) (end 148.4 58.8) (width 1) (layer "F.Cu") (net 11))
 (segment (start 162.8 75.8) (end 162.8 73.2) (width 1) (layer "F.Cu") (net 11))
 (segment (start 120.8 61.6) (end 122.394466 63.194466) (width 1) (layer "F.Cu") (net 11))
 (segment (start 122.394466 63.194466) (end 123.139466 63.194466) (width 1) (layer "F.Cu") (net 11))
 (segment (start 157.475 77.035) (end 155.035 77.035) (width 1) (layer "F.Cu") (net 12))
 (segment (start 155.035 77.035) (end 138.654466 60.654466) (width 1) (layer "F.Cu") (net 12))
 (segment (start 138.654466 60.654466) (end 123.139466 60.654466) (width 1) (layer "F.Cu") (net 12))
 (segment (start 131.935 135.865978) (end 133.200978 134.6) (width 1) (layer "B.Cu") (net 2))
 (segment (start 141.7 134.6) (end 150.12 126.18) (width 1) (layer "B.Cu") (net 2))
 (segment (start 131.935 136.425) (end 131.935 135.865978) (width 1) (layer "B.Cu") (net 2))
 (segment (start 150.12 126.18) (end 150.12 102.25) (width 1) (layer "B.Cu") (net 2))
 (segment (start 133.200978 134.6) (end 141.7 134.6) (width 1) (layer "B.Cu") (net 2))
 (segment (start 146.31 108.6) (end 152.66 102.25) (width 1) (layer "F.Cu") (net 7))
 (segment (start 131.935 132.875) (end 130.940148 131.880148) (width 1) (layer "F.Cu") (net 7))
 (segment (start 130.940148 121.409852) (end 143.75 108.6) (width 1) (layer "F.Cu") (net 7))
 (segment (start 130.940148 131.880148) (end 130.940148 121.409852) (width 1) (layer "F.Cu") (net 7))
 (segment (start 143.75 108.6) (end 146.31 108.6) (width 1) (layer "F.Cu") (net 7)))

